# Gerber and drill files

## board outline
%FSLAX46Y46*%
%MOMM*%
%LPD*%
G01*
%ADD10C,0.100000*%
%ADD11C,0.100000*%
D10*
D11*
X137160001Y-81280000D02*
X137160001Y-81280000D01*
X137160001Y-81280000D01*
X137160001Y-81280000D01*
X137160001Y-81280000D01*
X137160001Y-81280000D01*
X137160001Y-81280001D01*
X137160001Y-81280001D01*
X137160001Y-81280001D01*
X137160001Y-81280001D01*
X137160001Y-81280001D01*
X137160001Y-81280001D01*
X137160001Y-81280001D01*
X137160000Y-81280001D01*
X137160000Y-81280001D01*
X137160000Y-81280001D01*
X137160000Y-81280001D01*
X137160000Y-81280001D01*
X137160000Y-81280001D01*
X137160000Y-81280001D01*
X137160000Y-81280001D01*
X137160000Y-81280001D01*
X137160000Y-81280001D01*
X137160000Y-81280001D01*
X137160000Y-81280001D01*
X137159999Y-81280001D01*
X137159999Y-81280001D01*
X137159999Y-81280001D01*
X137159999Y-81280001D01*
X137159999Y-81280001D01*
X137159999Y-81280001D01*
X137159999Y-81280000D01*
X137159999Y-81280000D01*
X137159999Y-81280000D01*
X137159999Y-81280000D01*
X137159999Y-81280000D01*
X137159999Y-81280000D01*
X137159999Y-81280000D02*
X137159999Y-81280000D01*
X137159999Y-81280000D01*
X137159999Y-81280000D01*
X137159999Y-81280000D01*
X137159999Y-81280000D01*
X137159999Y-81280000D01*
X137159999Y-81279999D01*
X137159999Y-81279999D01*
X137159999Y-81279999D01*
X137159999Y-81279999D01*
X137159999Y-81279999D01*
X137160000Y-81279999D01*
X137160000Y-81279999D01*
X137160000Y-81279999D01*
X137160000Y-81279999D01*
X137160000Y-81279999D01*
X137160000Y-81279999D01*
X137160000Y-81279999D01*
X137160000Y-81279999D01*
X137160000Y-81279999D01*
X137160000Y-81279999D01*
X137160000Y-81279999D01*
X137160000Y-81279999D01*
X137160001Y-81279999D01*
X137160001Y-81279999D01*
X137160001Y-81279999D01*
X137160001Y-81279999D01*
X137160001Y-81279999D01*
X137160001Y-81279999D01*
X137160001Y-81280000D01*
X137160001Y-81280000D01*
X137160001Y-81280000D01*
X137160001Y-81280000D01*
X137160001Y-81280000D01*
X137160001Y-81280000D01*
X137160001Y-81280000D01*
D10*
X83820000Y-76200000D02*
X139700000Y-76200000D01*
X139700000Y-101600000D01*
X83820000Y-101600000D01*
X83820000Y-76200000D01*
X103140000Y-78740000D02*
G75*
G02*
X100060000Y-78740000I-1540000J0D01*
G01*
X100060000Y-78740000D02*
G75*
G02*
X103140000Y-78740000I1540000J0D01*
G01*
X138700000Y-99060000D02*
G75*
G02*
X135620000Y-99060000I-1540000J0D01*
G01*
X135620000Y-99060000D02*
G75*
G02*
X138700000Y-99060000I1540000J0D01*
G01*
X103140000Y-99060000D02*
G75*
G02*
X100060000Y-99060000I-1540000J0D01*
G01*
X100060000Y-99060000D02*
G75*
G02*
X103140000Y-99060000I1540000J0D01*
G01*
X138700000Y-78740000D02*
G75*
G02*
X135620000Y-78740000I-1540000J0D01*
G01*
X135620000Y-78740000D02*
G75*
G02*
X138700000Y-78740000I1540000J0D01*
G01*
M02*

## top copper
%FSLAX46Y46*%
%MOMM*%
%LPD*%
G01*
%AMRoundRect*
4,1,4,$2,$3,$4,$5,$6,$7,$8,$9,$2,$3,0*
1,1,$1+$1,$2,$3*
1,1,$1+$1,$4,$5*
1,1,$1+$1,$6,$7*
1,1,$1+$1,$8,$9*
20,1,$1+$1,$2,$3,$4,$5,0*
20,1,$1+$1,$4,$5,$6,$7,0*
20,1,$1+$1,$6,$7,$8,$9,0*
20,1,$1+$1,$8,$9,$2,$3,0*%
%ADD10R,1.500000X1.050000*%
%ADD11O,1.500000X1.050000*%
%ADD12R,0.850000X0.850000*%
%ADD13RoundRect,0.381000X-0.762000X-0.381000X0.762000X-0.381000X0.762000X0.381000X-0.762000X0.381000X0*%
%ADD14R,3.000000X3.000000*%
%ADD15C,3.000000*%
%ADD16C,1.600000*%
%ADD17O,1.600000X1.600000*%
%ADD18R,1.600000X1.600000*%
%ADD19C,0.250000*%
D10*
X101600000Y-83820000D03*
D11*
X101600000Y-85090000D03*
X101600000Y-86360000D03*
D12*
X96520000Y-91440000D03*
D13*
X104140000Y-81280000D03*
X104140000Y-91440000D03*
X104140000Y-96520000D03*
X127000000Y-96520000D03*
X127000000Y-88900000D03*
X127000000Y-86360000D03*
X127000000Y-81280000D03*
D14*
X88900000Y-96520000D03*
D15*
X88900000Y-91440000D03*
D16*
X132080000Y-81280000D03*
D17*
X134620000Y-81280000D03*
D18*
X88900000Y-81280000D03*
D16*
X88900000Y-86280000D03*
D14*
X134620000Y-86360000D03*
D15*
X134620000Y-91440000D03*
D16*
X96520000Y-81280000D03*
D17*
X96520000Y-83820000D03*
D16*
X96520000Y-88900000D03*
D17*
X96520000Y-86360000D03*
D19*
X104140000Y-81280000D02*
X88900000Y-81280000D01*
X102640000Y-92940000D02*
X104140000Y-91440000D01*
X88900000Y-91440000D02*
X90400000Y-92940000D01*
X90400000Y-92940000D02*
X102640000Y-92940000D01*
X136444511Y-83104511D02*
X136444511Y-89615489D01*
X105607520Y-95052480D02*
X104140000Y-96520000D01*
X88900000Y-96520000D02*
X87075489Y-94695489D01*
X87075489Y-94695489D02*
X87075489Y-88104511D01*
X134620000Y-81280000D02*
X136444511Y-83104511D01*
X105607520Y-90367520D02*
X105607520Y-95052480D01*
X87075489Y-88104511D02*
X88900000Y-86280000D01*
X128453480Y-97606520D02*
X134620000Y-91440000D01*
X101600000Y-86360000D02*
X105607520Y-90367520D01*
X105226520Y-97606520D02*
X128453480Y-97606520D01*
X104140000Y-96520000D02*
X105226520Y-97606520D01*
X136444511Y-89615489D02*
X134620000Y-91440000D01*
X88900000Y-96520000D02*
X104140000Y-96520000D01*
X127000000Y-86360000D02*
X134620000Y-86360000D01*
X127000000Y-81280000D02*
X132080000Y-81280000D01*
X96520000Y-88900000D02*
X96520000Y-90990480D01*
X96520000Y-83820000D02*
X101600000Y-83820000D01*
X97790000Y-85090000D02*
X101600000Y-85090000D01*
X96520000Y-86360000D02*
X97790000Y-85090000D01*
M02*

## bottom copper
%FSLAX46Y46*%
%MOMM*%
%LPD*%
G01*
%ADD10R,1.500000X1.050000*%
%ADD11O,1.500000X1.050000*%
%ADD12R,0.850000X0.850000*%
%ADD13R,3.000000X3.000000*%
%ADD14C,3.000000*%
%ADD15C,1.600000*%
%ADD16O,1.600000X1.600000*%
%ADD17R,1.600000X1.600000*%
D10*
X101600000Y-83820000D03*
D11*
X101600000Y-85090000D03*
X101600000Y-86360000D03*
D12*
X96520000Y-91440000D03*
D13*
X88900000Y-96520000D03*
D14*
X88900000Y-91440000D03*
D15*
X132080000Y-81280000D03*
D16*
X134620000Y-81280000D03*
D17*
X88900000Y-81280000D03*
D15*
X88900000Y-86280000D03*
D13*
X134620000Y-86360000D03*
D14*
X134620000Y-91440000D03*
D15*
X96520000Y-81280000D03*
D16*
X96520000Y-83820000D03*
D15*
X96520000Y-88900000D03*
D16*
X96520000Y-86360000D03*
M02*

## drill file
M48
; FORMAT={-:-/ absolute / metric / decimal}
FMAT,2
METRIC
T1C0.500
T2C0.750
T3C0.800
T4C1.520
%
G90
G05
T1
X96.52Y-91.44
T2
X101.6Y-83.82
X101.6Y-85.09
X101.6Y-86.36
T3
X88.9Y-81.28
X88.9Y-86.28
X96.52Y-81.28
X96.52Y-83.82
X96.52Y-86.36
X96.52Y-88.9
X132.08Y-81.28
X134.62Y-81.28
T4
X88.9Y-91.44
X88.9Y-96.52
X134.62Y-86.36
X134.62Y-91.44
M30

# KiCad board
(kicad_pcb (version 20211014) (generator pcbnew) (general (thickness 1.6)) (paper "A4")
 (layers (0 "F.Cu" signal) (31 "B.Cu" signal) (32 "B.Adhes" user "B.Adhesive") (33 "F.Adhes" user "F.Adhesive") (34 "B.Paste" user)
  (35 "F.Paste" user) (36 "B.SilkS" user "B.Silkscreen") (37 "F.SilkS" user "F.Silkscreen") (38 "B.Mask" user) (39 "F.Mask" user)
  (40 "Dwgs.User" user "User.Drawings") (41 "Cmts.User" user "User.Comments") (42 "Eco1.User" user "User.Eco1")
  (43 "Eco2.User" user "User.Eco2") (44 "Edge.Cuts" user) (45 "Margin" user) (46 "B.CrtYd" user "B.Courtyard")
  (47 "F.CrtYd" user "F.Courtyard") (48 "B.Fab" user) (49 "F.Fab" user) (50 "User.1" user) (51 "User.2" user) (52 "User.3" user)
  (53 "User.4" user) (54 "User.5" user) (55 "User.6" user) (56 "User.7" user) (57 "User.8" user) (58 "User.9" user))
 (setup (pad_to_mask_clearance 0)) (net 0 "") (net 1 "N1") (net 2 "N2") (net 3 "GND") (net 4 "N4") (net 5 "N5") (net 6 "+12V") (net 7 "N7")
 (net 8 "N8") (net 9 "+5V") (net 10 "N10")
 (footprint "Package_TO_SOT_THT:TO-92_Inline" (layer "F.Cu") (at 101.6 83.82 -90)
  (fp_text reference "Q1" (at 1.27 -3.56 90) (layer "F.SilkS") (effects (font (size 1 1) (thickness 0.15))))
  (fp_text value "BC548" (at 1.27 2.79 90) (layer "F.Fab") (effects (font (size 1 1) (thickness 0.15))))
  (pad "1" thru_hole rect (at 0 0 270) (size 1.05 1.5) (drill 0.75) (layers *.Cu *.Mask) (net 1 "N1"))
  (pad "2" thru_hole oval (at 1.27 0 270) (size 1.05 1.5) (drill 0.75) (layers *.Cu *.Mask) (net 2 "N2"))
  (pad "3" thru_hole oval (at 2.54 0 270) (size 1.05 1.5) (drill 0.75) (layers *.Cu *.Mask) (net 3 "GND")))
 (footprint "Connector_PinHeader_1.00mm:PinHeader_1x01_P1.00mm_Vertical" (layer "F.Cu") (at 96.52 91.44)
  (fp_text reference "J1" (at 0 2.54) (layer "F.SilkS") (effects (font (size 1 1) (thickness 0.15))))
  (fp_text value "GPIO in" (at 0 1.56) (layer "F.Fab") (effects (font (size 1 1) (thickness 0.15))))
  (pad "1" thru_hole rect (at 0 0) (size 0.85 0.85) (drill 0.5) (layers *.Cu *.Mask) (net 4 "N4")))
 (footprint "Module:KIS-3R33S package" (layer "F.Cu") (at 116.84 86.36)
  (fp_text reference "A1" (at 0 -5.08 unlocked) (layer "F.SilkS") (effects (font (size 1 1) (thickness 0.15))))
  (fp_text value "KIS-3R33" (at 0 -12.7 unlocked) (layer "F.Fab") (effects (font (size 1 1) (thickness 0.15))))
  (pad "1" smd roundrect (at -12.7 -5.08) (size 2.286 1.524) (layers "F.Cu" "F.Paste" "F.Mask") (roundrect_rratio 0.25) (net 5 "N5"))
  (pad "2" smd roundrect (at -12.7 5.08) (size 2.286 1.524) (layers "F.Cu" "F.Paste" "F.Mask") (roundrect_rratio 0.25) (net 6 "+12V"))
  (pad "3" smd roundrect (at -12.7 10.16) (size 2.286 1.524) (layers "F.Cu" "F.Paste" "F.Mask") (roundrect_rratio 0.25) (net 3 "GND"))
  (pad "4" smd roundrect (at 10.16 10.16) (size 2.286 1.524) (layers "F.Cu" "F.Paste" "F.Mask") (roundrect_rratio 0.25) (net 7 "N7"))
  (pad "5" smd roundrect (at 10.16 2.54) (size 2.286 1.524) (layers "F.Cu" "F.Paste" "F.Mask") (roundrect_rratio 0.25) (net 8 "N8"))
  (pad "6" smd roundrect (at 10.16 0) (size 2.286 1.524) (layers "F.Cu" "F.Paste" "F.Mask") (roundrect_rratio 0.25) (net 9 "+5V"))
  (pad "7" smd roundrect (at 10.16 -5.08) (size 2.286 1.524) (layers "F.Cu" "F.Paste" "F.Mask") (roundrect_rratio 0.25) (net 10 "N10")))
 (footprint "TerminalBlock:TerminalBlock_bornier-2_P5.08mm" (layer "F.Cu") (at 88.9 96.52 90)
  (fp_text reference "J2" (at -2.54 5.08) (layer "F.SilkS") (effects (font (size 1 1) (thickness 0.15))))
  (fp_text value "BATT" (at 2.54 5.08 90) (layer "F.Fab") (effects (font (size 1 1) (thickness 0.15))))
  (pad "1" thru_hole rect (at 0 0 90) (size 3 3) (drill 1.52) (layers *.Cu *.Mask) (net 3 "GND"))
  (pad "2" thru_hole circle (at 5.08 0 90) (size 3 3) (drill 1.52) (layers *.Cu *.Mask) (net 6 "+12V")))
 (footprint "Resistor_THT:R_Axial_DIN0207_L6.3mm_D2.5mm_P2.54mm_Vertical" (layer "F.Cu") (at 132.08 81.28)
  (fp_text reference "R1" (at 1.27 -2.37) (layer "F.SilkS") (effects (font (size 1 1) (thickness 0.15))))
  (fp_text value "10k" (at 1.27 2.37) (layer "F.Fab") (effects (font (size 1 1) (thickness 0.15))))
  (pad "1" thru_hole circle (at 0 0) (size 1.6 1.6) (drill 0.8) (layers *.Cu *.Mask) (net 10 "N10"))
  (pad "2" thru_hole oval (at 2.54 0) (size 1.6 1.6) (drill 0.8) (layers *.Cu *.Mask) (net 3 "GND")))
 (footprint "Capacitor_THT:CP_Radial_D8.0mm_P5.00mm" (layer "F.Cu") (at 88.9 81.28 -90)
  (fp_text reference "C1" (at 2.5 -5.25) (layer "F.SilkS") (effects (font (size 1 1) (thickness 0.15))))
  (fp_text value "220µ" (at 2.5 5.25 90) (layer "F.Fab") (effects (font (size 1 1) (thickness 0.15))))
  (pad "1" thru_hole rect (at 0 0 270) (size 1.6 1.6) (drill 0.8) (layers *.Cu *.Mask) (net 5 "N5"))
  (pad "2" thru_hole circle (at 5 0 270) (size 1.6 1.6) (drill 0.8) (layers *.Cu *.Mask) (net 3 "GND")))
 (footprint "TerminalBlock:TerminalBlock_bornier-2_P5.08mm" (layer "F.Cu") (at 134.62 86.36 -90)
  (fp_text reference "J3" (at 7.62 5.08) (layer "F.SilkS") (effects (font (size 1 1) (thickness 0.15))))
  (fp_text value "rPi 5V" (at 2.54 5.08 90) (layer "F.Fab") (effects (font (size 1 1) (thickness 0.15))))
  (pad "1" thru_hole rect (at 0 0 270) (size 3 3) (drill 1.52) (layers *.Cu *.Mask) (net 9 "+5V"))
  (pad "2" thru_hole circle (at 5.08 0 270) (size 3 3) (drill 1.52) (layers *.Cu *.Mask) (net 3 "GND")))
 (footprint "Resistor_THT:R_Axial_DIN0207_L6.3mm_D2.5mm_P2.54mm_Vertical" (layer "F.Cu") (at 96.52 81.28 -90)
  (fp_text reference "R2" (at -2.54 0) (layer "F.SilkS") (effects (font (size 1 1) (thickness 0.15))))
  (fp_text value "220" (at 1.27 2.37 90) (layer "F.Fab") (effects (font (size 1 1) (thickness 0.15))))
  (pad "1" thru_hole circle (at 0 0 270) (size 1.6 1.6) (drill 0.8) (layers *.Cu *.Mask) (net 5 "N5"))
  (pad "2" thru_hole oval (at 2.54 0 270) (size 1.6 1.6) (drill 0.8) (layers *.Cu *.Mask) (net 1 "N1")))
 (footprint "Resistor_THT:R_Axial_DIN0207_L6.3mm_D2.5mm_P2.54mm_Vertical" (layer "F.Cu") (at 96.52 88.9 90)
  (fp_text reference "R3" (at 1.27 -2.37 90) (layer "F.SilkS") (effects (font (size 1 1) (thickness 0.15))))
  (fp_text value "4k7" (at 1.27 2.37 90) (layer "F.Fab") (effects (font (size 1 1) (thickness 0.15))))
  (pad "1" thru_hole circle (at 0 0 90) (size 1.6 1.6) (drill 0.8) (layers *.Cu *.Mask) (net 4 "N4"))
  (pad "2" thru_hole oval (at 2.54 0 90) (size 1.6 1.6) (drill 0.8) (layers *.Cu *.Mask) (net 2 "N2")))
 (gr_circle (center 137.16 81.28) (end 137.16 81.28) (layer "Edge.Cuts") (width 0.1) (fill none))
 (gr_rect (start 83.82 76.2) (end 139.7 101.6) (layer "Edge.Cuts") (width 0.1) (fill none))
 (gr_circle (center 101.6 78.74) (end 103.14 78.74) (layer "Edge.Cuts") (width 0.1) (fill none))
 (gr_circle (center 137.16 99.06) (end 138.7 99.06) (layer "Edge.Cuts") (width 0.1) (fill none))
 (gr_circle (center 101.6 99.06) (end 103.14 99.06) (layer "Edge.Cuts") (width 0.1) (fill none))
 (gr_circle (center 137.16 78.74) (end 138.7 78.74) (layer "Edge.Cuts") (width 0.1) (fill none))
 (segment (start 104.14 81.28) (end 88.9 81.28) (width 0.25) (layer "F.Cu") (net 5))
 (segment (start 102.64 92.94) (end 104.14 91.44) (width 0.25) (layer "F.Cu") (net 6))
 (segment (start 88.9 91.44) (end 90.4 92.94) (width 0.25) (layer "F.Cu") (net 6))
 (segment (start 90.4 92.94) (end 102.64 92.94) (width 0.25) (layer "F.Cu") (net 6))
 (segment (start 136.444511 83.104511) (end 136.444511 89.615489) (width 0.25) (layer "F.Cu") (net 3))
 (segment (start 105.60752 95.05248) (end 104.14 96.52) (width 0.25) (layer "F.Cu") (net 3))
 (segment (start 88.9 96.52) (end 87.075489 94.695489) (width 0.25) (layer "F.Cu") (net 3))
 (segment (start 87.075489 94.695489) (end 87.075489 88.104511) (width 0.25) (layer "F.Cu") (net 3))
 (segment (start 134.62 81.28) (end 136.444511 83.104511) (width 0.25) (layer "F.Cu") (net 3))
 (segment (start 105.60752 90.36752) (end 105.60752 95.05248) (width 0.25) (layer "F.Cu") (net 3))
 (segment (start 87.075489 88.104511) (end 88.9 86.28) (width 0.25) (layer "F.Cu") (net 3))
 (segment (start 128.45348 97.60652) (end 134.62 91.44) (width 0.25) (layer "F.Cu") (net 3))
 (segment (start 101.6 86.36) (end 105.60752 90.36752) (width 0.25) (layer "F.Cu") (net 3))
 (segment (start 105.22652 97.60652) (end 128.45348 97.60652) (width 0.25) (layer "F.Cu") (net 3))
 (segment (start 104.14 96.52) (end 105.22652 97.60652) (width 0.25) (layer "F.Cu") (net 3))
 (segment (start 136.444511 89.615489) (end 134.62 91.44) (width 0.25) (layer "F.Cu") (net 3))
 (segment (start 88.9 96.52) (end 104.14 96.52) (width 0.25) (layer "F.Cu") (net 3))
 (segment (start 127 86.36) (end 134.62 86.36) (width 0.25) (layer "F.Cu") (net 9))
 (segment (start 127 81.28) (end 132.08 81.28) (width 0.25) (layer "F.Cu") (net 10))
 (segment (start 96.52 88.9) (end 96.52 90.99048) (width 0.25) (layer "F.Cu") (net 4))
 (segment (start 96.52 83.82) (end 101.6 83.82) (width 0.25) (layer "F.Cu") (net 1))
 (segment (start 97.79 85.09) (end 101.6 85.09) (width 0.25) (layer "F.Cu") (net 2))
 (segment (start 96.52 86.36) (end 97.79 85.09) (width 0.25) (layer "F.Cu") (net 2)))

